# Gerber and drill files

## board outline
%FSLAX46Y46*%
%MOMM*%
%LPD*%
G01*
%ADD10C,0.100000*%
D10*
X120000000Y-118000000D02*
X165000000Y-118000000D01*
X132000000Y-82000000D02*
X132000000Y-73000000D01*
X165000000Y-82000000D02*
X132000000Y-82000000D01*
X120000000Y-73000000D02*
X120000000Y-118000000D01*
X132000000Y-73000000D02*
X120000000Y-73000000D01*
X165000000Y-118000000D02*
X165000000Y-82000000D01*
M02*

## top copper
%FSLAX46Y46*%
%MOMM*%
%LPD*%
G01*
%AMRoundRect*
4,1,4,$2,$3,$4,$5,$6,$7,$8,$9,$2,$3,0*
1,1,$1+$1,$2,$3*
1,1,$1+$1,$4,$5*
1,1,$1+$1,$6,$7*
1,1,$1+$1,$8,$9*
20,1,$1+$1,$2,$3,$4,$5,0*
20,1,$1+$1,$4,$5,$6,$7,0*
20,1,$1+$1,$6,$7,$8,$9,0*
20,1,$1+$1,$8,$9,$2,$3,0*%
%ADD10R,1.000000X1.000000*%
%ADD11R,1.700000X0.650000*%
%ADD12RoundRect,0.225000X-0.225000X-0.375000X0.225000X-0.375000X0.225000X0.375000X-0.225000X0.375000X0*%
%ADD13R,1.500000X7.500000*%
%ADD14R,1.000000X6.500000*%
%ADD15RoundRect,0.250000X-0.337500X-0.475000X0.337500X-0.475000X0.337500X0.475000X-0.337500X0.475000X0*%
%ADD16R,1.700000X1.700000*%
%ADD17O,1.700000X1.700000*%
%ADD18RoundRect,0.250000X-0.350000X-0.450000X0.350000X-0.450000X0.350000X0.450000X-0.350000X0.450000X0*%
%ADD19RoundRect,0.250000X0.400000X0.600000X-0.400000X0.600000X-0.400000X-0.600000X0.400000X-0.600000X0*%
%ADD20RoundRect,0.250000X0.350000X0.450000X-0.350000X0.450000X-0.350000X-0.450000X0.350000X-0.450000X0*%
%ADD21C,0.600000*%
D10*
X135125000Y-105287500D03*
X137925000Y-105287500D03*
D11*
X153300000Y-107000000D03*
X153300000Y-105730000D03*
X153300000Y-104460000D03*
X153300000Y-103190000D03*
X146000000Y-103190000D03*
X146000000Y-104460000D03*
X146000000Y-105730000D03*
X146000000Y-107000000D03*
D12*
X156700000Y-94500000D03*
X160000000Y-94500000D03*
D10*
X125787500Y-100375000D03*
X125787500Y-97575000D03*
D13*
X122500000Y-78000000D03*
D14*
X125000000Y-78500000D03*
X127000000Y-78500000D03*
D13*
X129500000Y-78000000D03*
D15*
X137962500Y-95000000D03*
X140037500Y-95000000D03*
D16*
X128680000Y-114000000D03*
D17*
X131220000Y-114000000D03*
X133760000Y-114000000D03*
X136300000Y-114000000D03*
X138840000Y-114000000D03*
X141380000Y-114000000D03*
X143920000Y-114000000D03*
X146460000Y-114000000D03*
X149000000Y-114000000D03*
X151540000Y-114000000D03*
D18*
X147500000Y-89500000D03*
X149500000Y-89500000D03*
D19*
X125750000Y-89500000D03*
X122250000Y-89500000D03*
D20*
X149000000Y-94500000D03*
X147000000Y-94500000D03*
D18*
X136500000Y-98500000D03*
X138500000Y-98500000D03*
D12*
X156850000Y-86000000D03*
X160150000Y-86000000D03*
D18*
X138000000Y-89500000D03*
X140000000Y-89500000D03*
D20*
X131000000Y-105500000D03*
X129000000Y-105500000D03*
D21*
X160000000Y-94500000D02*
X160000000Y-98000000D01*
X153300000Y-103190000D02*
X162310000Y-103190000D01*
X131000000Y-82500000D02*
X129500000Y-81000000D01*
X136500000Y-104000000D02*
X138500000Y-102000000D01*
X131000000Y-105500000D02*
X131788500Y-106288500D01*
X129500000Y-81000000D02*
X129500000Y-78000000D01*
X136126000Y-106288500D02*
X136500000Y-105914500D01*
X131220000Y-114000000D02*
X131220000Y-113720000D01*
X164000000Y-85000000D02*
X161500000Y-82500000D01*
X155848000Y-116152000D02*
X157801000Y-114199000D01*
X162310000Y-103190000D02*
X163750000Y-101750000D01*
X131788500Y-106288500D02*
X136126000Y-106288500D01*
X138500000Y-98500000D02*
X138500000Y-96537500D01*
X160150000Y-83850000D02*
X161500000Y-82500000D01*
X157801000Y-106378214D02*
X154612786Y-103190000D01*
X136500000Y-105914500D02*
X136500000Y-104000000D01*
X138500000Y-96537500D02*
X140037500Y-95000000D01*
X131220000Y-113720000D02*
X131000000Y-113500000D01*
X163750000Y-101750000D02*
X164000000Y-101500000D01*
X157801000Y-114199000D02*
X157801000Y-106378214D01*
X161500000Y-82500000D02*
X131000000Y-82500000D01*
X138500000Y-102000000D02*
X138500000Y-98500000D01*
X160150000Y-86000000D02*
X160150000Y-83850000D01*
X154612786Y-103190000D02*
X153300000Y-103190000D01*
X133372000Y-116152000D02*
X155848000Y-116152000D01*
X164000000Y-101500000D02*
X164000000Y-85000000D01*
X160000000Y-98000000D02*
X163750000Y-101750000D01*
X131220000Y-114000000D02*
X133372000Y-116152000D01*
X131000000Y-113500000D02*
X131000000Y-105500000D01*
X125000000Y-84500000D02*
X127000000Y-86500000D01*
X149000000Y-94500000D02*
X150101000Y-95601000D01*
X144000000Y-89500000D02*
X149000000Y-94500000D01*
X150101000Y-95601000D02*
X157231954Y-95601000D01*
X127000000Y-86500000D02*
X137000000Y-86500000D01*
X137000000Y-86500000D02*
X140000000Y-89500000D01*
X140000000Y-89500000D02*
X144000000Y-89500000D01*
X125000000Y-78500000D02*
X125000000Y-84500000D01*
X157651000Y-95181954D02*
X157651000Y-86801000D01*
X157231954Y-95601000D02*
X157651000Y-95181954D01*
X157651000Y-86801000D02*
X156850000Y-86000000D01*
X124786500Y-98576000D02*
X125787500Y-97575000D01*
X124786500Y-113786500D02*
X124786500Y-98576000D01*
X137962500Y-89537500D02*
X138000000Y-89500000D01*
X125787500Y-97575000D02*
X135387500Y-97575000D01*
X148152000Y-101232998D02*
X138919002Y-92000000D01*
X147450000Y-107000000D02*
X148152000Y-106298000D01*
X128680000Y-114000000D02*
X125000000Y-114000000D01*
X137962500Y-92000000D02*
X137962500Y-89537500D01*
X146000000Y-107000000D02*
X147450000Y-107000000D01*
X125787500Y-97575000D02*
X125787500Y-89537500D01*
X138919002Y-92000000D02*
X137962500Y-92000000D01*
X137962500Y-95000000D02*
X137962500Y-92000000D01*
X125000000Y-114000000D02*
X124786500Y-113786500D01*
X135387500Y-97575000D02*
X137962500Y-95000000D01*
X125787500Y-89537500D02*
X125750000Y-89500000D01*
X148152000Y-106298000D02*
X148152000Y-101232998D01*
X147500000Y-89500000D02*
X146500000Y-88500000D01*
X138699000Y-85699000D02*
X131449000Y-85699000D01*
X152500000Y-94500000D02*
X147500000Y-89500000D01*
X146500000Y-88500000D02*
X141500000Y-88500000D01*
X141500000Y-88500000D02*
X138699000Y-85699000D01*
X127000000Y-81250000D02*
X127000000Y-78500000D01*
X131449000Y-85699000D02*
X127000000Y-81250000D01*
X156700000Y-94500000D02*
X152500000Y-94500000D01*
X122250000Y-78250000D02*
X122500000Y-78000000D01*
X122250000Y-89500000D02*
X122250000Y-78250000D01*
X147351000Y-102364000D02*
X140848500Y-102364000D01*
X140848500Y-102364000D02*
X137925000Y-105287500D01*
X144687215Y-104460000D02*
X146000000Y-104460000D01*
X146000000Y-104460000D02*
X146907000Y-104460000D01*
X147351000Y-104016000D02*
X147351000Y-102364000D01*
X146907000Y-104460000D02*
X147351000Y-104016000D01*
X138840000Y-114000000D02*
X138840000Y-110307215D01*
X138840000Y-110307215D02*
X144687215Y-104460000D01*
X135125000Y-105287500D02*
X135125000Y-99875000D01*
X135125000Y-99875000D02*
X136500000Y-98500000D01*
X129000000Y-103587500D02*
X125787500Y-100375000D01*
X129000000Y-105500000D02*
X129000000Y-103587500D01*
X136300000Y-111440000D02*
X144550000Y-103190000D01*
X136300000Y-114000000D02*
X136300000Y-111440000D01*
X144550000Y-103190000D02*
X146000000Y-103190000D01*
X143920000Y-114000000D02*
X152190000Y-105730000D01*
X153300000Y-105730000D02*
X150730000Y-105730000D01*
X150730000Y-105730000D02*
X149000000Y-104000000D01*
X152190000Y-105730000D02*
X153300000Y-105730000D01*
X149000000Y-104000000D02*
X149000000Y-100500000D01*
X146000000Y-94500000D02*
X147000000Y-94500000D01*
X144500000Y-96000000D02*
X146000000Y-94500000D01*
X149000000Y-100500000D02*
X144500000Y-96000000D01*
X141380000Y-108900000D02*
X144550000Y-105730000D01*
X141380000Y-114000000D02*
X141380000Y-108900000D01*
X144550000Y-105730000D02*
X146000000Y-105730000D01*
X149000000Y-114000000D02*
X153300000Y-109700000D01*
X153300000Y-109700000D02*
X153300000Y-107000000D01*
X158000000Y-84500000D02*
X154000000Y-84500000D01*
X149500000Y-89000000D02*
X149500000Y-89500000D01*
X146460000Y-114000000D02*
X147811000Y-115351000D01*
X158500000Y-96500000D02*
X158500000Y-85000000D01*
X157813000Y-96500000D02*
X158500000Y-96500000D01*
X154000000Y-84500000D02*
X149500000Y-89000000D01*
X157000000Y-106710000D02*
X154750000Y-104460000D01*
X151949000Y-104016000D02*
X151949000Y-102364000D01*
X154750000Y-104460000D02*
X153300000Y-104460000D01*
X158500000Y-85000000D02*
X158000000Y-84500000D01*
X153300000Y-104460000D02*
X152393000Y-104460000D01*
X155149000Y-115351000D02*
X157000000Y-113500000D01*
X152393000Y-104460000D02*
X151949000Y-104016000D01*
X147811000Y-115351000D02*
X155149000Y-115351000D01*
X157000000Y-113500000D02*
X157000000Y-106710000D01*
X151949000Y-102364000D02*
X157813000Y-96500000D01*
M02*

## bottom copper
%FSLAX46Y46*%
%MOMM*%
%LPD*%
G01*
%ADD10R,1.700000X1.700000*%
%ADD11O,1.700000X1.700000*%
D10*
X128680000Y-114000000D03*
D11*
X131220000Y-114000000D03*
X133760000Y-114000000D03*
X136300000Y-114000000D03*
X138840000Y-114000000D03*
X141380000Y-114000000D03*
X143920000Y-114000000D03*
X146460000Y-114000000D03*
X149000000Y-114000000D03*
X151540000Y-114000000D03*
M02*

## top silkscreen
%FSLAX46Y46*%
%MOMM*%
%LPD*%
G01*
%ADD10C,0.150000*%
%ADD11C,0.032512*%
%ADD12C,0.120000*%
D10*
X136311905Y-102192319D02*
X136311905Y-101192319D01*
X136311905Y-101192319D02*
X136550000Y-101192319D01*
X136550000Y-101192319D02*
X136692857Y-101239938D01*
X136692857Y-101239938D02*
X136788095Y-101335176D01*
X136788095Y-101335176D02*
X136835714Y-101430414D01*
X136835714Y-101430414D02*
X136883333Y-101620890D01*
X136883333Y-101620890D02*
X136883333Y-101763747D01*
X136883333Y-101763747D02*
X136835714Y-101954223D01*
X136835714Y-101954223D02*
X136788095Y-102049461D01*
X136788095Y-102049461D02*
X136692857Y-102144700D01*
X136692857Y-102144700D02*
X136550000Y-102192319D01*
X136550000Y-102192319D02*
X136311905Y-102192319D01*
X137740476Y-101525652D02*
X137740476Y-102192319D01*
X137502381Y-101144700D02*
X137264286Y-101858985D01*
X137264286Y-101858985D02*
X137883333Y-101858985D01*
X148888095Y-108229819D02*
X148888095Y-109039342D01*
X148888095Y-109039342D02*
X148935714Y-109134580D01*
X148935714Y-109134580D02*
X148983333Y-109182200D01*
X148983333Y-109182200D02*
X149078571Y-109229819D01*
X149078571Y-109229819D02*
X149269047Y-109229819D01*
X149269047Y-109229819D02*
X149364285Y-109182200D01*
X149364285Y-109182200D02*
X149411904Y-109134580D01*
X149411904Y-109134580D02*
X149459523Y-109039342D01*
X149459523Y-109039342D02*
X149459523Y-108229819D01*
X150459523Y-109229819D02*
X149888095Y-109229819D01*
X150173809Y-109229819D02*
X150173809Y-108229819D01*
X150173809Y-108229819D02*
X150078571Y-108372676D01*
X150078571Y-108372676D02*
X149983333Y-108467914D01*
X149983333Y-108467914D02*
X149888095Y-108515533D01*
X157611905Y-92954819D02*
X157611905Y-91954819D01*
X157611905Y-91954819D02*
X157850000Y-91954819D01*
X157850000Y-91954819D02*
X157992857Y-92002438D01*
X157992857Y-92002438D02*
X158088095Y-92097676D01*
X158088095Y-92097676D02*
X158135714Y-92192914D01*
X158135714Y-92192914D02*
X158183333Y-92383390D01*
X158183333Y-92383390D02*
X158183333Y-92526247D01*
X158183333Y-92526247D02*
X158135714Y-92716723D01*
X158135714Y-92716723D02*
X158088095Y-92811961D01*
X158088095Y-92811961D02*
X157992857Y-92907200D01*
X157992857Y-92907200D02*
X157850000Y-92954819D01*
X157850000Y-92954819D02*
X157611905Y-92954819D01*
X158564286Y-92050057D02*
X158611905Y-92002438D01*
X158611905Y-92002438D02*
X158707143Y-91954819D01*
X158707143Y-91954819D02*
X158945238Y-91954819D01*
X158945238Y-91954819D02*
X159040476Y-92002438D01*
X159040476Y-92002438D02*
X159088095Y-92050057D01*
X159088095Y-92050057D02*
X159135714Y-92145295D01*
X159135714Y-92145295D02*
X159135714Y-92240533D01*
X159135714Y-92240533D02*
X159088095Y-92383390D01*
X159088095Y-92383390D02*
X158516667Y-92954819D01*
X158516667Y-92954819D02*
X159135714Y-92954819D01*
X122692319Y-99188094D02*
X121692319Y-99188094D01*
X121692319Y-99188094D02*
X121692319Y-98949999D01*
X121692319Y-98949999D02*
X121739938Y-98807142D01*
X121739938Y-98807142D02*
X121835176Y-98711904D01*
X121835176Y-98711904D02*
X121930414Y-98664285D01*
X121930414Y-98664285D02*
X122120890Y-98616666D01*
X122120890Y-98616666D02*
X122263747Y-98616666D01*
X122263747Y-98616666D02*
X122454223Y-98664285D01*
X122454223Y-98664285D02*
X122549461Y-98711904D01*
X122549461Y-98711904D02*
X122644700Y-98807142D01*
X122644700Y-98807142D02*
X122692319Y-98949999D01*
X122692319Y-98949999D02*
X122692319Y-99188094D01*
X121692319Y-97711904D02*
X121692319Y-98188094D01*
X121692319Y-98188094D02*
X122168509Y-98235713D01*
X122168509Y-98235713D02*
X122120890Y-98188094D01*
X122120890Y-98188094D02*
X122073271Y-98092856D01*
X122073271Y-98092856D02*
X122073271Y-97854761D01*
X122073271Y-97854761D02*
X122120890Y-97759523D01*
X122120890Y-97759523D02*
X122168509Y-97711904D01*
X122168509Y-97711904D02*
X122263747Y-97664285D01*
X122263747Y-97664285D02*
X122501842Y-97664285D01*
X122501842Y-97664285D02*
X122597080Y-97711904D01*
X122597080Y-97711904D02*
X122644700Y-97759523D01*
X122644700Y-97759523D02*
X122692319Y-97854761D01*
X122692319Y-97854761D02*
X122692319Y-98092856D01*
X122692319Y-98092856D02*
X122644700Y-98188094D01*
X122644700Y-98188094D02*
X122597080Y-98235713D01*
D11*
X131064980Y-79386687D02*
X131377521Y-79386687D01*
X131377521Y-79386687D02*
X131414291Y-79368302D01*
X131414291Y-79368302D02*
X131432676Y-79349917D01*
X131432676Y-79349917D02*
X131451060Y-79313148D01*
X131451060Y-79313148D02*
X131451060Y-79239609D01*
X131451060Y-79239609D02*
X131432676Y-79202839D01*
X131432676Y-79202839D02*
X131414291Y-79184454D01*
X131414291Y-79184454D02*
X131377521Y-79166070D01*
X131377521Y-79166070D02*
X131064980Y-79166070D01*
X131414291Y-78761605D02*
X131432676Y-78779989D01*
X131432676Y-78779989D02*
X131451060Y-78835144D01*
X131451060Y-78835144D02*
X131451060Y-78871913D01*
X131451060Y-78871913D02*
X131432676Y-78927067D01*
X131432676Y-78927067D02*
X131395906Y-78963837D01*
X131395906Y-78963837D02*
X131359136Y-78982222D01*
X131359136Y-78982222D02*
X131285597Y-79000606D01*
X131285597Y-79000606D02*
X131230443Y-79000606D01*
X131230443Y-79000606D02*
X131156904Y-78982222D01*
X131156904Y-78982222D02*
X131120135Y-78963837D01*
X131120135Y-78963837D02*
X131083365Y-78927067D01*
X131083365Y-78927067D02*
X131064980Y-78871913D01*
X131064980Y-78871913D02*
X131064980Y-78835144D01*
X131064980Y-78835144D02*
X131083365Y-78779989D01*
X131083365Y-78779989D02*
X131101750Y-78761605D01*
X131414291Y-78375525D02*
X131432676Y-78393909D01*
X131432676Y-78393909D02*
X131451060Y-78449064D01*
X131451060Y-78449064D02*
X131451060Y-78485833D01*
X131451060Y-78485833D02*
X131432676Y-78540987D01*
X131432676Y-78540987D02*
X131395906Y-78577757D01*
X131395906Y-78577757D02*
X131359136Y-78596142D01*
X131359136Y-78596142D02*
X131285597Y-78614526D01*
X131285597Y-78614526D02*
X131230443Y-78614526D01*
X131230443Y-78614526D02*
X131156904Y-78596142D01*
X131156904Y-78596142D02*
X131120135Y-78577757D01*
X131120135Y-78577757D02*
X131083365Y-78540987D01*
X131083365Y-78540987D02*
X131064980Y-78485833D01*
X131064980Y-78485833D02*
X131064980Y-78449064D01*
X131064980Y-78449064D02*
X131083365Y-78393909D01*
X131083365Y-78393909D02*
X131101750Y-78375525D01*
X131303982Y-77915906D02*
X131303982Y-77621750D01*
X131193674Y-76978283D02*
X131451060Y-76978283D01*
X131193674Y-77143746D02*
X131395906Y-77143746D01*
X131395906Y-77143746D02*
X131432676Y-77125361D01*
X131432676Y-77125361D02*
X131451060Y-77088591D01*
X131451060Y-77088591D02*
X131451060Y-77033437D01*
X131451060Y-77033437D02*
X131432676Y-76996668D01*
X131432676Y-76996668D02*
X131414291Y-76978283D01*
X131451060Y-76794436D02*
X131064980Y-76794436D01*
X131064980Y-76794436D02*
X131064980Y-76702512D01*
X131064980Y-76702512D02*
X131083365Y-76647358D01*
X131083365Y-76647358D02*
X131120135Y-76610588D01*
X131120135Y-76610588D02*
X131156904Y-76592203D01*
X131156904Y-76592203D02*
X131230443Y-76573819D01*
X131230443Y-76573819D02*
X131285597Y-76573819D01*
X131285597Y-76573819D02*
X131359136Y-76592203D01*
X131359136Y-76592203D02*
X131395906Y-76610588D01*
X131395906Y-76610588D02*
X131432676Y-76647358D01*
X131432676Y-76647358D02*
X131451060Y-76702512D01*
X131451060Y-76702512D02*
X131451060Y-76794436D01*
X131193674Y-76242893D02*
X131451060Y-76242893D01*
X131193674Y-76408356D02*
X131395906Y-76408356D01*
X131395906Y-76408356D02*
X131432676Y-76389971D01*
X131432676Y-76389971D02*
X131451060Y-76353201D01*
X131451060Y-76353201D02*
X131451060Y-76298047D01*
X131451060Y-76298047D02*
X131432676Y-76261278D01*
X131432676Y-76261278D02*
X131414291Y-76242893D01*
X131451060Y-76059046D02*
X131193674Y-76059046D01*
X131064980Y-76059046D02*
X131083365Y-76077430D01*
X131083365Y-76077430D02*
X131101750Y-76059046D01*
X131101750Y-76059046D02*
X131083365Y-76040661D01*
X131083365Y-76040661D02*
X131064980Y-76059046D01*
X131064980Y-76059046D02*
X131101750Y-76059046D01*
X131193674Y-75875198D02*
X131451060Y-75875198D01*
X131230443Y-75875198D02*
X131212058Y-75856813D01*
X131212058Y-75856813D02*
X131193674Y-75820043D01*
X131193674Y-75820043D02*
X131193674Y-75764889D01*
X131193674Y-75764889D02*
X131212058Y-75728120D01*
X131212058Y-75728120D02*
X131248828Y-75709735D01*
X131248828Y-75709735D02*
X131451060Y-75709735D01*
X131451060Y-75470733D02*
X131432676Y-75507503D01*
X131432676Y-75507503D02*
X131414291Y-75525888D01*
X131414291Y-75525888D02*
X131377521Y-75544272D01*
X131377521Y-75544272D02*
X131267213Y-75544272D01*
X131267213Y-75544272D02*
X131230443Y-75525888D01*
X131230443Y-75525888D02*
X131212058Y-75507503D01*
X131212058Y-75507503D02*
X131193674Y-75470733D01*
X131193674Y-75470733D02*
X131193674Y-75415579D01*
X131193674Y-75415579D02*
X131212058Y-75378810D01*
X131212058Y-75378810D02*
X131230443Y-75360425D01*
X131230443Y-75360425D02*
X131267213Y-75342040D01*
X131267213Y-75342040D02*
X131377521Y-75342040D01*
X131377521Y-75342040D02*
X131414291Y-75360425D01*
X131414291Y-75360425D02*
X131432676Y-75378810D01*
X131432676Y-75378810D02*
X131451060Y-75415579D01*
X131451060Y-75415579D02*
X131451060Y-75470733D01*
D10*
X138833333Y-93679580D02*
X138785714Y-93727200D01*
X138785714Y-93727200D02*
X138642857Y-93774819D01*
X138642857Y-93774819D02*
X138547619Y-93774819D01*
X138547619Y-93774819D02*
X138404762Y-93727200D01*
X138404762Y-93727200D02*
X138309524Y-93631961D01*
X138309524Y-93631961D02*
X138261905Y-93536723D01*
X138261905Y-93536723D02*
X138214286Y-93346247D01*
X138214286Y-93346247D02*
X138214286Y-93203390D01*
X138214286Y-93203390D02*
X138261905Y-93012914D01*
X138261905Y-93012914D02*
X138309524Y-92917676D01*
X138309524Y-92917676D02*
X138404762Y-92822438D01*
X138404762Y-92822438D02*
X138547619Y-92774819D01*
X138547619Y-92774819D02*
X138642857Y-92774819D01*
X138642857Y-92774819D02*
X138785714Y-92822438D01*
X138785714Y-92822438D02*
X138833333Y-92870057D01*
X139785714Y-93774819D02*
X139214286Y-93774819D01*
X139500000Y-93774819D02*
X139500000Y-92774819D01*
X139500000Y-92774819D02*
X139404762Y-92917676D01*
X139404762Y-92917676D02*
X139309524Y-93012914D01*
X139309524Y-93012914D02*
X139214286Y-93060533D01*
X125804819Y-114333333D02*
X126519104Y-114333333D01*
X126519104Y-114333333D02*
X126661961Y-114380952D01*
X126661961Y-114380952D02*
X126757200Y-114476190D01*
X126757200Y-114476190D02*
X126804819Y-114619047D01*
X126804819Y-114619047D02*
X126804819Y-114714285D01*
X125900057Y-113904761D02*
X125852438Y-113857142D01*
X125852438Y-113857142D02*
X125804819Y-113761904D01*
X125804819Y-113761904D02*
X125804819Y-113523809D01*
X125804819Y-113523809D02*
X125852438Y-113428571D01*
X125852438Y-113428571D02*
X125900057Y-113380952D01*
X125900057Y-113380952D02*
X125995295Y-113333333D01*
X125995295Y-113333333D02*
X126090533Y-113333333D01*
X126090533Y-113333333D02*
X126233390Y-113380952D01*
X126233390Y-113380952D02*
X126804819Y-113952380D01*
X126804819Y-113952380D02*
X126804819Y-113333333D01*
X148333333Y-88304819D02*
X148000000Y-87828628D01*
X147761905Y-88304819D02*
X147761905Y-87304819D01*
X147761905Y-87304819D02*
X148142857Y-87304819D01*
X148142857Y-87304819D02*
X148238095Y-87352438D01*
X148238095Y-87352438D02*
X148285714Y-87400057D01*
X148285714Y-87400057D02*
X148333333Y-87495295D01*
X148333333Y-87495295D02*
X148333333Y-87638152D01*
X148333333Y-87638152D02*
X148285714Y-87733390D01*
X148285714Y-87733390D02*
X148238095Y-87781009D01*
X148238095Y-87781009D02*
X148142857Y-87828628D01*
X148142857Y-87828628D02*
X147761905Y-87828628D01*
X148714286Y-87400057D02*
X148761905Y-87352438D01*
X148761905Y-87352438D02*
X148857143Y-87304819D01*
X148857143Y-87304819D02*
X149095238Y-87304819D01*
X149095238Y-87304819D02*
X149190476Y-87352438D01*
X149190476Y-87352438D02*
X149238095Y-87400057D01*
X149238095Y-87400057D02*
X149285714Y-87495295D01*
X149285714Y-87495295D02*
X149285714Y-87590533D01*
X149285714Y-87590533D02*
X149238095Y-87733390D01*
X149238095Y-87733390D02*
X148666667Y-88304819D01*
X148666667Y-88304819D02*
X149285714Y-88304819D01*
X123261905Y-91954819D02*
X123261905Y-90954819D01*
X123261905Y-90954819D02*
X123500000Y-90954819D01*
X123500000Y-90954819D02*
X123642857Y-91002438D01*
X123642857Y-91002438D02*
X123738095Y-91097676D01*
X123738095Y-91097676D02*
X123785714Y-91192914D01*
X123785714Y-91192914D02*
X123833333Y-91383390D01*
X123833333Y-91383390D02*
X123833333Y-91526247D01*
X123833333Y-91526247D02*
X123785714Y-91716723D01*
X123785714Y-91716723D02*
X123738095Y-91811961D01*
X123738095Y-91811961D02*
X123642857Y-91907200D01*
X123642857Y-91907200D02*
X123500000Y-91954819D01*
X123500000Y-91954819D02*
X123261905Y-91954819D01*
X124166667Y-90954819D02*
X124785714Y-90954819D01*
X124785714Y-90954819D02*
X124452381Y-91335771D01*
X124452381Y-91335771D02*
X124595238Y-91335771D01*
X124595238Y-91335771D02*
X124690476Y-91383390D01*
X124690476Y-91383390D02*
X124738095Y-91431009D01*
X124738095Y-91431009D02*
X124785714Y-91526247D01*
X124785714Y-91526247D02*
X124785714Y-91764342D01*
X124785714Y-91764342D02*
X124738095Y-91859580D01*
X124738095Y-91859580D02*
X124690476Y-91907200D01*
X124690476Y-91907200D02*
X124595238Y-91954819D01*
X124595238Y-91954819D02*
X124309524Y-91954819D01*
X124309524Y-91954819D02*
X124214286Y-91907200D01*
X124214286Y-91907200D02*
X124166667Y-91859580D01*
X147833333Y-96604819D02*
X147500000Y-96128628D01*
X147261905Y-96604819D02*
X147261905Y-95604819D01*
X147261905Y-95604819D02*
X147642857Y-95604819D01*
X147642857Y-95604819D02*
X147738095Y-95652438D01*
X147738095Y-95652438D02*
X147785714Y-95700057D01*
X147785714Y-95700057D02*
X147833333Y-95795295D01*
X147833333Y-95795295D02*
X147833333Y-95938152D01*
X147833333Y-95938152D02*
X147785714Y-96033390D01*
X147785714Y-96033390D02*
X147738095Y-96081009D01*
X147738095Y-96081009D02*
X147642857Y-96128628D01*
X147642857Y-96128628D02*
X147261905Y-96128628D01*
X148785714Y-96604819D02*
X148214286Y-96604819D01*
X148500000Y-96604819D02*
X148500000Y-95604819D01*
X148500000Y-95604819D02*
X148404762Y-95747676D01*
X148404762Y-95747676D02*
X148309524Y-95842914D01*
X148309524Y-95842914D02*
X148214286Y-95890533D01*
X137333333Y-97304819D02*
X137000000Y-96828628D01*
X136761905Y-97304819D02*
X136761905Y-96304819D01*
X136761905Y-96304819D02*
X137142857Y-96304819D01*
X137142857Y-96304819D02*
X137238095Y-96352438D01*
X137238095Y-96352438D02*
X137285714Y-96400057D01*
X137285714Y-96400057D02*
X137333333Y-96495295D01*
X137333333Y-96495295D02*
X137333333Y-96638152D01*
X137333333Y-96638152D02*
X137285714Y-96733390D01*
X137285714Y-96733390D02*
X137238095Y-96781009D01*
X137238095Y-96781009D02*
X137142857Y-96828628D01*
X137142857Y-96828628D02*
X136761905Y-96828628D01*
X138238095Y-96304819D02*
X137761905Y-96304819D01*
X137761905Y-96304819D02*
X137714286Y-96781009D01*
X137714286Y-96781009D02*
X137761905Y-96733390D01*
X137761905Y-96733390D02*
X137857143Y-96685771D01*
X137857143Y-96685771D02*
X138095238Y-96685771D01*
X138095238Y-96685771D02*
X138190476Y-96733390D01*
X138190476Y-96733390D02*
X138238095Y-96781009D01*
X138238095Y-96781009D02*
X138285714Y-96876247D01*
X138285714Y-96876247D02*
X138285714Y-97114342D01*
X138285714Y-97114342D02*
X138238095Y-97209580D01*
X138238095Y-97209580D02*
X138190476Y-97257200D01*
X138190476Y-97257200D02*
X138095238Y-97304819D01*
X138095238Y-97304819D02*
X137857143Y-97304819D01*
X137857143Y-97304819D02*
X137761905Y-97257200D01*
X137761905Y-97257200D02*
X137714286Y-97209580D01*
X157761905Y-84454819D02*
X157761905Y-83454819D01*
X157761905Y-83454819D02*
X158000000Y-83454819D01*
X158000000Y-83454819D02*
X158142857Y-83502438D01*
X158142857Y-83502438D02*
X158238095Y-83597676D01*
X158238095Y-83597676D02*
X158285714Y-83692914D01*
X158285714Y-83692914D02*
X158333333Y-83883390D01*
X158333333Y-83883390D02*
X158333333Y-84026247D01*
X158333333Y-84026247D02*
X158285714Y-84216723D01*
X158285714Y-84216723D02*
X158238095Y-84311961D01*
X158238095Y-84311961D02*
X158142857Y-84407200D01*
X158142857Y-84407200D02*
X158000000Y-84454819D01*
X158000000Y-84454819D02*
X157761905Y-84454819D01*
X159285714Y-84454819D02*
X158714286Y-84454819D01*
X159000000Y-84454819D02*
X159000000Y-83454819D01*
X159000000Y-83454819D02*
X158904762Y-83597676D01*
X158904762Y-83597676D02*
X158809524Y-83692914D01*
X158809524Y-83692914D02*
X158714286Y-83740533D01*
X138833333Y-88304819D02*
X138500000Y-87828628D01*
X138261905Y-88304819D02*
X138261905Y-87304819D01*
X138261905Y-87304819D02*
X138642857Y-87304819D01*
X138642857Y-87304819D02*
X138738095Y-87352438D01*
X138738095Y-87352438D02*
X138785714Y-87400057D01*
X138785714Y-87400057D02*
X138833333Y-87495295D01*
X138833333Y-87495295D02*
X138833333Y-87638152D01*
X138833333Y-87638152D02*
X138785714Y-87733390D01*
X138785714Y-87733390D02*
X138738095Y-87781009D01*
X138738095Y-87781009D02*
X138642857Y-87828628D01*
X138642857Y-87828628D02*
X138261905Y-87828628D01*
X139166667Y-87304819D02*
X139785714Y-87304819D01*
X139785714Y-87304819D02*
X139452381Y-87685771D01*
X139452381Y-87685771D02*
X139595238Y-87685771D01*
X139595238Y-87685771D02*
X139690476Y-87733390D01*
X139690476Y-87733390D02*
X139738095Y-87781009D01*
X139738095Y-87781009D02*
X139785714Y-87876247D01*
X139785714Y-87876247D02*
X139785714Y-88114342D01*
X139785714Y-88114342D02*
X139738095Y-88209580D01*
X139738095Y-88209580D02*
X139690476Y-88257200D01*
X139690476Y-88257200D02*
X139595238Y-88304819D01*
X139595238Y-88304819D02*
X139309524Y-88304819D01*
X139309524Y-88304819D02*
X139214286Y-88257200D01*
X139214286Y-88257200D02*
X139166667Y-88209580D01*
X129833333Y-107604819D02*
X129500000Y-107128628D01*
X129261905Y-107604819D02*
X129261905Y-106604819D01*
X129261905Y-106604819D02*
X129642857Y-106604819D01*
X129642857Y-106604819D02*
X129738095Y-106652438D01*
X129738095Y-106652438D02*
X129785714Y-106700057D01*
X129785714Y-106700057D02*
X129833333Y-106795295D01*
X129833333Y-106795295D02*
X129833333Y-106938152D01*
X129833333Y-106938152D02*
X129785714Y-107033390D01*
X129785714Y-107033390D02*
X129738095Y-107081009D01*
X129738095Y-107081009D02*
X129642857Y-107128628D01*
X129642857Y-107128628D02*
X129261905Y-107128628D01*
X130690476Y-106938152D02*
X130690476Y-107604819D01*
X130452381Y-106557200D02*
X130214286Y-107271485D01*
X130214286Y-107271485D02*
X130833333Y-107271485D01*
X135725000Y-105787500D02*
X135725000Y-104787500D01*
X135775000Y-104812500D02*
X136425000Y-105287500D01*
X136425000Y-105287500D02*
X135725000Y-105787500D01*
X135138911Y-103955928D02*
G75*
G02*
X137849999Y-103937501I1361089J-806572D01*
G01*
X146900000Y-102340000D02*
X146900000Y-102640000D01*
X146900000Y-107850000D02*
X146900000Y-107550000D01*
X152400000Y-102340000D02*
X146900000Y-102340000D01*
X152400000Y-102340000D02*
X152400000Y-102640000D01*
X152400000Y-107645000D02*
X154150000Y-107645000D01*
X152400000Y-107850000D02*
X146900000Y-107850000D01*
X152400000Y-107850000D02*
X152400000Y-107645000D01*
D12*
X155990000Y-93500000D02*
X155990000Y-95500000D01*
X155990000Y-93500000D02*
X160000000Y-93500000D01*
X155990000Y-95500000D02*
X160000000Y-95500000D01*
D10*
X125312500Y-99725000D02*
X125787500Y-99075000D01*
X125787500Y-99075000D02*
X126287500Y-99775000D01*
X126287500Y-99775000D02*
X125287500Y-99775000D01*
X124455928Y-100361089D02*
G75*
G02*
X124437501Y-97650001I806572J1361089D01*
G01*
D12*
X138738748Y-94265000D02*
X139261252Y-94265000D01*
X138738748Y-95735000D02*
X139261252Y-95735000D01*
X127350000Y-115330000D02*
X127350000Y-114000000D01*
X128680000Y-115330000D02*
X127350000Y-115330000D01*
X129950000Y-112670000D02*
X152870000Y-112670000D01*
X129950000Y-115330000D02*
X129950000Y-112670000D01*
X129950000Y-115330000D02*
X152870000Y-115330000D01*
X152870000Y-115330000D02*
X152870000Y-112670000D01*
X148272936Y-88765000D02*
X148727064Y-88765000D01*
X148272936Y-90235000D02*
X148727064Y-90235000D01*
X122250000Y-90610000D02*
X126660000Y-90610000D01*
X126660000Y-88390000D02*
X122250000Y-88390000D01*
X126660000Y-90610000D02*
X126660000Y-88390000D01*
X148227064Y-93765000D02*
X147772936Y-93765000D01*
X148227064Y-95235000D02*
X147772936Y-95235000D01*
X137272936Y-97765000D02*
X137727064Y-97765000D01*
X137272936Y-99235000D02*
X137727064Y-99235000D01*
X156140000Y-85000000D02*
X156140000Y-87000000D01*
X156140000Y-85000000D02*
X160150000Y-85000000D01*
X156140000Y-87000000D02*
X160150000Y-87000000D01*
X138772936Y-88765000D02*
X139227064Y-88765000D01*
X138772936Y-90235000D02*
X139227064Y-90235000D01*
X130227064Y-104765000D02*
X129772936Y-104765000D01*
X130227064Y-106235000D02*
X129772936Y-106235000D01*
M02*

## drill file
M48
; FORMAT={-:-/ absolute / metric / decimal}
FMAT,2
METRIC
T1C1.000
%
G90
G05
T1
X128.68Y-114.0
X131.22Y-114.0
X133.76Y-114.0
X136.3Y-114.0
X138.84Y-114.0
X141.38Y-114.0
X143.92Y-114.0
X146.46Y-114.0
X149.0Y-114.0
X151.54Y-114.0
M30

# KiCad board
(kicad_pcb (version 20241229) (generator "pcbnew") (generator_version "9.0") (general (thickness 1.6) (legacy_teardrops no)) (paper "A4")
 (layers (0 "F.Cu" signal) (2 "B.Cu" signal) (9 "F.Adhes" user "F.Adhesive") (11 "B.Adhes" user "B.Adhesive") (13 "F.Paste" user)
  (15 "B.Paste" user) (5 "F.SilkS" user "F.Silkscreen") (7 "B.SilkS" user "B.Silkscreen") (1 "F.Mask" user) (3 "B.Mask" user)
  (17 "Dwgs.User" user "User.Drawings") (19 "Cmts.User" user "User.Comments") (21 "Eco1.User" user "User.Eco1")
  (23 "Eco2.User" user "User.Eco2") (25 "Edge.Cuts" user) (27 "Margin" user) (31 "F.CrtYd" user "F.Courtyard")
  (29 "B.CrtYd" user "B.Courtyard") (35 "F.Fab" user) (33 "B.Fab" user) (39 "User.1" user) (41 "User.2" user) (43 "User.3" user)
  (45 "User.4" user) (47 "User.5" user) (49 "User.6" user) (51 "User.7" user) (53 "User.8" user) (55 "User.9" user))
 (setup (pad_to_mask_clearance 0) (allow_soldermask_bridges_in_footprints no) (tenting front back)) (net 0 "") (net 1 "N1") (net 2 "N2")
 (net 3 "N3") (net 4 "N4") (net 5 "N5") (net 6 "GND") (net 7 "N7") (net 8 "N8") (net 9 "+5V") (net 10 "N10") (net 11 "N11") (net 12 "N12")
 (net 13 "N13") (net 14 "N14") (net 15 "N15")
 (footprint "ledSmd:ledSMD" (layer "F.Cu") (at 136.925 105.2875)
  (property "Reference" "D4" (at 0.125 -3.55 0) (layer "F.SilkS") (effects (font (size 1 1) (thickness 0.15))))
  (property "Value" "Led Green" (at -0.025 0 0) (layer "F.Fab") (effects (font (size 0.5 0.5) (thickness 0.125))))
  (fp_line (start -1.2 0.5) (end -1.2 -0.5) (stroke (width 0.15) (type solid)) (layer "F.SilkS"))
  (fp_line (start -1.15 -0.475) (end -0.5 0) (stroke (width 0.15) (type solid)) (layer "F.SilkS"))
  (fp_line (start -0.5 0) (end -1.2 0.5) (stroke (width 0.15) (type solid)) (layer "F.SilkS"))
  (fp_arc (start -1.786089 -1.331572) (mid -0.435753 -2.107089) (end 0.924999 -1.349999) (stroke (width 0.15) (type solid))
   (layer "F.SilkS"))
  (pad "1" smd rect (at -1.8 0) (size 1 1) (layers "F.Cu" "F.Mask" "F.Paste") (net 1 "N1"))
  (pad "2" smd rect (at 1 0) (size 1 1) (layers "F.Cu" "F.Mask" "F.Paste") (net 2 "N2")))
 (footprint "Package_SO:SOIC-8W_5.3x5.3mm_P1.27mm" (layer "F.Cu") (at 149.65 105.095 180)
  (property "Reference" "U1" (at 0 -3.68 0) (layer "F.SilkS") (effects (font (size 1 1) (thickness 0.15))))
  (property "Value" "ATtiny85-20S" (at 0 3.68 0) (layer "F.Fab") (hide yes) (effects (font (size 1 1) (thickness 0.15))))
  (fp_line (start 2.75 2.755) (end 2.75 2.455) (stroke (width 0.15) (type solid)) (layer "F.SilkS"))
  (fp_line (start 2.75 -2.755) (end 2.75 -2.455) (stroke (width 0.15) (type solid)) (layer "F.SilkS"))
  (fp_line (start -2.75 2.755) (end 2.75 2.755) (stroke (width 0.15) (type solid)) (layer "F.SilkS"))
  (fp_line (start -2.75 2.755) (end -2.75 2.455) (stroke (width 0.15) (type solid)) (layer "F.SilkS"))
  (fp_line (start -2.75 -2.55) (end -4.5 -2.55) (stroke (width 0.15) (type solid)) (layer "F.SilkS"))
  (fp_line (start -2.75 -2.755) (end 2.75 -2.755) (stroke (width 0.15) (type solid)) (layer "F.SilkS"))
  (fp_line (start -2.75 -2.755) (end -2.75 -2.55) (stroke (width 0.15) (type solid)) (layer "F.SilkS"))
  (pad "1" smd rect (at -3.65 -1.905 180) (size 1.7 0.65) (layers "F.Cu" "F.Mask" "F.Paste") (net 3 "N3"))
  (pad "2" smd rect (at -3.65 -0.635 180) (size 1.7 0.65) (layers "F.Cu" "F.Mask" "F.Paste") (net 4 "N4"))
  (pad "3" smd rect (at -3.65 0.635 180) (size 1.7 0.65) (layers "F.Cu" "F.Mask" "F.Paste") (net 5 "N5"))
  (pad "4" smd rect (at -3.65 1.905 180) (size 1.7 0.65) (layers "F.Cu" "F.Mask" "F.Paste") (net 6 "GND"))
  (pad "5" smd rect (at 3.65 1.905 180) (size 1.7 0.65) (layers "F.Cu" "F.Mask" "F.Paste") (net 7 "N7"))
  (pad "6" smd rect (at 3.65 0.635 180) (size 1.7 0.65) (layers "F.Cu" "F.Mask" "F.Paste") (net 2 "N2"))
  (pad "7" smd rect (at 3.65 -0.635 180) (size 1.7 0.65) (layers "F.Cu" "F.Mask" "F.Paste") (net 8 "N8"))
  (pad "8" smd rect (at 3.65 -1.905 180) (size 1.7 0.65) (layers "F.Cu" "F.Mask" "F.Paste") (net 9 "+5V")))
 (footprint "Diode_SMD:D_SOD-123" (layer "F.Cu") (at 158.35 94.5)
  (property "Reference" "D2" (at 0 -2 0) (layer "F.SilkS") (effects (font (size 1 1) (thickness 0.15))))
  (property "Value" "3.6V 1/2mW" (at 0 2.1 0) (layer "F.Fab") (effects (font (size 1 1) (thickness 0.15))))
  (fp_line (start -2.36 -1) (end -2.36 1) (stroke (width 0.12) (type solid)) (layer "F.SilkS"))
  (fp_line (start -2.36 -1) (end 1.65 -1) (stroke (width 0.12) (type solid)) (layer "F.SilkS"))
  (fp_line (start -2.36 1) (end 1.65 1) (stroke (width 0.12) (type solid)) (layer "F.SilkS"))
  (pad "1" smd roundrect (at -1.65 0) (size 0.9 1.2) (layers "F.Cu" "F.Mask" "F.Paste") (roundrect_rratio 0.25) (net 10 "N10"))
  (pad "2" smd roundrect (at 1.65 0) (size 0.9 1.2) (layers "F.Cu" "F.Mask" "F.Paste") (roundrect_rratio 0.25) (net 6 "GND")))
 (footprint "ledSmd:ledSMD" (layer "F.Cu") (at 125.7875 98.575 90)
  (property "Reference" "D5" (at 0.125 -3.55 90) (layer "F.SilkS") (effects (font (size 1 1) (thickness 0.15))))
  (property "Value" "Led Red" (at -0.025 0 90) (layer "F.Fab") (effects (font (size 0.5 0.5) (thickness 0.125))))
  (fp_line (start -1.15 -0.475) (end -0.5 0) (stroke (width 0.15) (type solid)) (layer "F.SilkS"))
  (fp_line (start -0.5 0) (end -1.2 0.5) (stroke (width 0.15) (type solid)) (layer "F.SilkS"))
  (fp_line (start -1.2 0.5) (end -1.2 -0.5) (stroke (width 0.15) (type solid)) (layer "F.SilkS"))
  (fp_arc (start -1.786089 -1.331572) (mid -0.435753 -2.107089) (end 0.924999 -1.349999) (stroke (width 0.15) (type solid))
   (layer "F.SilkS"))
  (pad "1" smd rect (at -1.8 0 90) (size 1 1) (layers "F.Cu" "F.Mask" "F.Paste") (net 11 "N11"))
  (pad "2" smd rect (at 1 0 90) (size 1 1) (layers "F.Cu" "F.Mask" "F.Paste") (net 9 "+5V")))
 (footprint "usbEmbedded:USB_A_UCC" (layer "F.Cu") (at 126 78.2 -90)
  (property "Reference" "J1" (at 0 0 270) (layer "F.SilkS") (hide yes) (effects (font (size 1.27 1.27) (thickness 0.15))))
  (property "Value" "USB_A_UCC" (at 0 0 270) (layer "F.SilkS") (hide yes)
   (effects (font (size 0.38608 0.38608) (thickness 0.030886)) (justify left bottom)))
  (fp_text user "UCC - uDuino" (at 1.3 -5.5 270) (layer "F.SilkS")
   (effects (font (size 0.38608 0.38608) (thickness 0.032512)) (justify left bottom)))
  (pad "1" smd rect (at -0.2 3.5 270) (size 7.5 1.5) (layers "F.Cu" "F.Mask" "F.Paste") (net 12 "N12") (solder_mask_margin 0.1016))
  (pad "2" smd rect (at 0.3 1 270) (size 6.5 1) (layers "F.Cu" "F.Mask" "F.Paste") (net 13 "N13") (solder_mask_margin 0.1016))
  (pad "3" smd rect (at 0.3 -1 270) (size 6.5 1) (layers "F.Cu" "F.Mask" "F.Paste") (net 10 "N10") (solder_mask_margin 0.1016))
  (pad "4" smd rect (at -0.2 -3.5 270) (size 7.5 1.5) (layers "F.Cu" "F.Mask" "F.Paste") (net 6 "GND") (solder_mask_margin 0.1016)))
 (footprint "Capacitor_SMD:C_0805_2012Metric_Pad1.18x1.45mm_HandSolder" (layer "F.Cu") (at 139 95)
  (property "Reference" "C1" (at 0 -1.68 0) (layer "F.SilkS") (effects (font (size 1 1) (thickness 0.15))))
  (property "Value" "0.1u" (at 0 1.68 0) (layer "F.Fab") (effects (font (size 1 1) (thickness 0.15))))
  (fp_line (start -0.261252 -0.735) (end 0.261252 -0.735) (stroke (width 0.12) (type solid)) (layer "F.SilkS"))
  (fp_line (start -0.261252 0.735) (end 0.261252 0.735) (stroke (width 0.12) (type solid)) (layer "F.SilkS"))
  (pad "1" smd roundrect (at -1.0375 0) (size 1.175 1.45) (layers "F.Cu" "F.Mask" "F.Paste") (roundrect_rratio 0.212766) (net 9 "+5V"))
  (pad "2" smd roundrect (at 1.0375 0) (size 1.175 1.45) (layers "F.Cu" "F.Mask" "F.Paste") (roundrect_rratio 0.212766) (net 6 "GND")))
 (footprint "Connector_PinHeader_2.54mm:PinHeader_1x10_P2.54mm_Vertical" (layer "F.Cu") (at 128.68 114 90)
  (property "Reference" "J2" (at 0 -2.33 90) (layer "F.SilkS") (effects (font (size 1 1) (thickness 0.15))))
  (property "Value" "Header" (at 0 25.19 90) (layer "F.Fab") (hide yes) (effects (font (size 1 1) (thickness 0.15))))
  (fp_line (start -1.33 -1.33) (end 0 -1.33) (stroke (width 0.12) (type solid)) (layer "F.SilkS"))
  (fp_line (start -1.33 0) (end -1.33 -1.33) (stroke (width 0.12) (type solid)) (layer "F.SilkS"))
  (fp_line (start 1.33 1.27) (end 1.33 24.19) (stroke (width 0.12) (type solid)) (layer "F.SilkS"))
  (fp_line (start -1.33 1.27) (end 1.33 1.27) (stroke (width 0.12) (type solid)) (layer "F.SilkS"))
  (fp_line (start -1.33 1.27) (end -1.33 24.19) (stroke (width 0.12) (type solid)) (layer "F.SilkS"))
  (fp_line (start -1.33 24.19) (end 1.33 24.19) (stroke (width 0.12) (type solid)) (layer "F.SilkS"))
  (pad "1" thru_hole rect (at 0 0 90) (size 1.7 1.7) (drill 1) (layers "*.Cu" "*.Mask") (remove_unused_layers no) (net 9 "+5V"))
  (pad "2" thru_hole oval (at 0 2.54 90) (size 1.7 1.7) (drill 1) (layers "*.Cu" "*.Mask") (remove_unused_layers no) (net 6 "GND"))
  (pad "3" thru_hole oval (at 0 5.08 90) (size 1.7 1.7) (drill 1) (layers "*.Cu" "*.Mask") (remove_unused_layers no) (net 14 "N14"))
  (pad "4" thru_hole oval (at 0 7.62 90) (size 1.7 1.7) (drill 1) (layers "*.Cu" "*.Mask") (remove_unused_layers no) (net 7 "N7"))
  (pad "5" thru_hole oval (at 0 10.16 90) (size 1.7 1.7) (drill 1) (layers "*.Cu" "*.Mask") (remove_unused_layers no) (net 2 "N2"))
  (pad "6" thru_hole oval (at 0 12.7 90) (size 1.7 1.7) (drill 1) (layers "*.Cu" "*.Mask") (remove_unused_layers no) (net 8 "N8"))
  (pad "7" thru_hole oval (at 0 15.24 90) (size 1.7 1.7) (drill 1) (layers "*.Cu" "*.Mask") (remove_unused_layers no) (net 4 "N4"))
  (pad "8" thru_hole oval (at 0 17.78 90) (size 1.7 1.7) (drill 1) (layers "*.Cu" "*.Mask") (remove_unused_layers no) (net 5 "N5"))
  (pad "9" thru_hole oval (at 0 20.32 90) (size 1.7 1.7) (drill 1) (layers "*.Cu" "*.Mask") (remove_unused_layers no) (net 3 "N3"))
  (pad "10" thru_hole oval (at 0 22.86 90) (size 1.7 1.7) (drill 1) (layers "*.Cu" "*.Mask") (remove_unused_layers no) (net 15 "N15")))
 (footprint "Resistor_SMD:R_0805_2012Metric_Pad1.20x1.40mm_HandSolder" (layer "F.Cu") (at 148.5 89.5)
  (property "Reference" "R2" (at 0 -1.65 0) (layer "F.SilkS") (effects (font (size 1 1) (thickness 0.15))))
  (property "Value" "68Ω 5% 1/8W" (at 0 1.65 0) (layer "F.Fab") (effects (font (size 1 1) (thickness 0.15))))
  (fp_line (start -0.227064 -0.735) (end 0.227064 -0.735) (stroke (width 0.12) (type solid)) (layer "F.SilkS"))
  (fp_line (start -0.227064 0.735) (end 0.227064 0.735) (stroke (width 0.12) (type solid)) (layer "F.SilkS"))
  (pad "1" smd roundrect (at -1 0) (size 1.2 1.4) (layers "F.Cu" "F.Mask" "F.Paste") (roundrect_rratio 0.208333) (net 10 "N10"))
  (pad "2" smd roundrect (at 1 0) (size 1.2 1.4) (layers "F.Cu" "F.Mask" "F.Paste") (roundrect_rratio 0.208333) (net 5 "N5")))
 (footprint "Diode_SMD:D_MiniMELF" (layer "F.Cu") (at 124 89.5 180)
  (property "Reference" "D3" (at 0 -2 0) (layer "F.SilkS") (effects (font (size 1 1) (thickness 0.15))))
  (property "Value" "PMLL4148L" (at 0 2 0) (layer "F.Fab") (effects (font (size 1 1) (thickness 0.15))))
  (fp_line (start 1.75 -1.11) (end -2.66 -1.11) (stroke (width 0.12) (type solid)) (layer "F.SilkS"))
  (fp_line (start -2.66 1.11) (end 1.75 1.11) (stroke (width 0.12) (type solid)) (layer "F.SilkS"))
  (fp_line (start -2.66 -1.11) (end -2.66 1.11) (stroke (width 0.12) (type solid)) (layer "F.SilkS"))
  (pad "1" smd roundrect (at -1.75 0 180) (size 1.3 1.7) (layers "F.Cu" "F.Mask" "F.Paste") (roundrect_rratio 0.1923076923) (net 9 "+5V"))
  (pad "2" smd roundrect (at 1.75 0 180) (size 1.3 1.7) (layers "F.Cu" "F.Mask" "F.Paste") (roundrect_rratio 0.1923076923) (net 12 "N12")))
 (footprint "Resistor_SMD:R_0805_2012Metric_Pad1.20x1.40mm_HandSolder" (layer "F.Cu") (at 148 94.5 180)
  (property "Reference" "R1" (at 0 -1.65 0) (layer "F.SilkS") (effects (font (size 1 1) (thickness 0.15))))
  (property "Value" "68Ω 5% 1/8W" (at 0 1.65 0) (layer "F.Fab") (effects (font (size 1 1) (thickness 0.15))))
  (fp_line (start -0.227064 0.735) (end 0.227064 0.735) (stroke (width 0.12) (type solid)) (layer "F.SilkS"))
  (fp_line (start -0.227064 -0.735) (end 0.227064 -0.735) (stroke (width 0.12) (type solid)) (layer "F.SilkS"))
  (pad "1" smd roundrect (at -1 0 180) (size 1.2 1.4) (layers "F.Cu" "F.Mask" "F.Paste") (roundrect_rratio 0.208333) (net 13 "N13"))
  (pad "2" smd roundrect (at 1 0 180) (size 1.2 1.4) (layers "F.Cu" "F.Mask" "F.Paste") (roundrect_rratio 0.208333) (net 4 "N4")))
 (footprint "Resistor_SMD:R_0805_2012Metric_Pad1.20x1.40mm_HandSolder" (layer "F.Cu") (at 137.5 98.5)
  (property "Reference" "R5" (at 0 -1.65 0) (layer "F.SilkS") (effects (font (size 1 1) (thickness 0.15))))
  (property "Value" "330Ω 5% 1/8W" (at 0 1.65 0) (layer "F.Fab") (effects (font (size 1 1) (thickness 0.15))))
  (fp_line (start -0.227064 -0.735) (end 0.227064 -0.735) (stroke (width 0.12) (type solid)) (layer "F.SilkS"))
  (fp_line (start -0.227064 0.735) (end 0.227064 0.735) (stroke (width 0.12) (type solid)) (layer "F.SilkS"))
  (pad "1" smd roundrect (at -1 0) (size 1.2 1.4) (layers "F.Cu" "F.Mask" "F.Paste") (roundrect_rratio 0.208333) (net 1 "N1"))
  (pad "2" smd roundrect (at 1 0) (size 1.2 1.4) (layers "F.Cu" "F.Mask" "F.Paste") (roundrect_rratio 0.208333) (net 6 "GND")))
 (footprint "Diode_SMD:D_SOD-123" (layer "F.Cu") (at 158.5 86)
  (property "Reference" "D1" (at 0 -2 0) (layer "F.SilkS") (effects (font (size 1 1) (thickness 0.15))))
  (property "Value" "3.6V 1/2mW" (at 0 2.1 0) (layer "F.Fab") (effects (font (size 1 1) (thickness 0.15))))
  (fp_line (start -2.36 -1) (end -2.36 1) (stroke (width 0.12) (type solid)) (layer "F.SilkS"))
  (fp_line (start -2.36 -1) (end 1.65 -1) (stroke (width 0.12) (type solid)) (layer "F.SilkS"))
  (fp_line (start -2.36 1) (end 1.65 1) (stroke (width 0.12) (type solid)) (layer "F.SilkS"))
  (pad "1" smd roundrect (at -1.65 0) (size 0.9 1.2) (layers "F.Cu" "F.Mask" "F.Paste") (roundrect_rratio 0.25) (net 13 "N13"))
  (pad "2" smd roundrect (at 1.65 0) (size 0.9 1.2) (layers "F.Cu" "F.Mask" "F.Paste") (roundrect_rratio 0.25) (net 6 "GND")))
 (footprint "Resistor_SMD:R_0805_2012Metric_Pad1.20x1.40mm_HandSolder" (layer "F.Cu") (at 139 89.5)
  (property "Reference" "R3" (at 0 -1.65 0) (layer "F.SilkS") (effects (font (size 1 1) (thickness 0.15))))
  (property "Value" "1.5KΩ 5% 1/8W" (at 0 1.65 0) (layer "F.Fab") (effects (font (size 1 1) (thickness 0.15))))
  (fp_line (start -0.227064 -0.735) (end 0.227064 -0.735) (stroke (width 0.12) (type solid)) (layer "F.SilkS"))
  (fp_line (start -0.227064 0.735) (end 0.227064 0.735) (stroke (width 0.12) (type solid)) (layer "F.SilkS"))
  (pad "1" smd roundrect (at -1 0) (size 1.2 1.4) (layers "F.Cu" "F.Mask" "F.Paste") (roundrect_rratio 0.208333) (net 9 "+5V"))
  (pad "2" smd roundrect (at 1 0) (size 1.2 1.4) (layers "F.Cu" "F.Mask" "F.Paste") (roundrect_rratio 0.208333) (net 13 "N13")))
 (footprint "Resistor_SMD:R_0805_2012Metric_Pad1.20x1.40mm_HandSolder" (layer "F.Cu") (at 130 105.5 180)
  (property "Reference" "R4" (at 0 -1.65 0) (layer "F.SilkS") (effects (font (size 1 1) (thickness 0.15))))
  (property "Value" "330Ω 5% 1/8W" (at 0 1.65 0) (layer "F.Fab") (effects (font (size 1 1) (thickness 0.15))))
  (fp_line (start -0.227064 0.735) (end 0.227064 0.735) (stroke (width 0.12) (type solid)) (layer "F.SilkS"))
  (fp_line (start -0.227064 -0.735) (end 0.227064 -0.735) (stroke (width 0.12) (type solid)) (layer "F.SilkS"))
  (pad "1" smd roundrect (at -1 0 180) (size 1.2 1.4) (layers "F.Cu" "F.Mask" "F.Paste") (roundrect_rratio 0.208333) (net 6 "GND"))
  (pad "2" smd roundrect (at 1 0 180) (size 1.2 1.4) (layers "F.Cu" "F.Mask" "F.Paste") (roundrect_rratio 0.208333) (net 11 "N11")))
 (gr_line (start 120 118) (end 165 118) (stroke (width 0.1) (type default)) (layer "Edge.Cuts"))
 (gr_line (start 132 82) (end 132 73) (stroke (width 0.1) (type default)) (layer "Edge.Cuts"))
 (gr_line (start 165 82) (end 132 82) (stroke (width 0.1) (type default)) (layer "Edge.Cuts"))
 (gr_line (start 120 73) (end 120 118) (stroke (width 0.1) (type default)) (layer "Edge.Cuts"))
 (gr_line (start 132 73) (end 120 73) (stroke (width 0.1) (type default)) (layer "Edge.Cuts"))
 (gr_line (start 165 118) (end 165 82) (stroke (width 0.1) (type default)) (layer "Edge.Cuts"))
 (segment (start 160 94.5) (end 160 98) (width 0.6) (layer "F.Cu") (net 6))
 (segment (start 153.3 103.19) (end 162.31 103.19) (width 0.6) (layer "F.Cu") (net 6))
 (segment (start 131 82.5) (end 129.5 81) (width 0.6) (layer "F.Cu") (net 6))
 (segment (start 136.5 104) (end 138.5 102) (width 0.6) (layer "F.Cu") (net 6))
 (segment (start 131 105.5) (end 131.7885 106.2885) (width 0.6) (layer "F.Cu") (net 6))
 (segment (start 129.5 81) (end 129.5 78) (width 0.6) (layer "F.Cu") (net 6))
 (segment (start 136.126 106.2885) (end 136.5 105.9145) (width 0.6) (layer "F.Cu") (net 6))
 (segment (start 131.22 114) (end 131.22 113.72) (width 0.6) (layer "F.Cu") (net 6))
 (segment (start 164 85) (end 161.5 82.5) (width 0.6) (layer "F.Cu") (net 6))
 (segment (start 155.848 116.152) (end 157.801 114.199) (width 0.6) (layer "F.Cu") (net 6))
 (segment (start 162.31 103.19) (end 163.75 101.75) (width 0.6) (layer "F.Cu") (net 6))
 (segment (start 131.7885 106.2885) (end 136.126 106.2885) (width 0.6) (layer "F.Cu") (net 6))
 (segment (start 138.5 98.5) (end 138.5 96.5375) (width 0.6) (layer "F.Cu") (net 6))
 (segment (start 160.15 83.85) (end 161.5 82.5) (width 0.6) (layer "F.Cu") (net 6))
 (segment (start 157.801 106.378214) (end 154.612786 103.19) (width 0.6) (layer "F.Cu") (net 6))
 (segment (start 136.5 105.9145) (end 136.5 104) (width 0.6) (layer "F.Cu") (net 6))
 (segment (start 138.5 96.5375) (end 140.0375 95) (width 0.6) (layer "F.Cu") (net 6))
 (segment (start 131.22 113.72) (end 131 113.5) (width 0.6) (layer "F.Cu") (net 6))
 (segment (start 163.75 101.75) (end 164 101.5) (width 0.6) (layer "F.Cu") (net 6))
 (segment (start 157.801 114.199) (end 157.801 106.378214) (width 0.6) (layer "F.Cu") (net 6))
 (segment (start 161.5 82.5) (end 131 82.5) (width 0.6) (layer "F.Cu") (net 6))
 (segment (start 138.5 102) (end 138.5 98.5) (width 0.6) (layer "F.Cu") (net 6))
 (segment (start 160.15 86) (end 160.15 83.85) (width 0.6) (layer "F.Cu") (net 6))
 (segment (start 154.612786 103.19) (end 153.3 103.19) (width 0.6) (layer "F.Cu") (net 6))
 (segment (start 133.372 116.152) (end 155.848 116.152) (width 0.6) (layer "F.Cu") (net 6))
 (segment (start 164 101.5) (end 164 85) (width 0.6) (layer "F.Cu") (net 6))
 (segment (start 160 98) (end 163.75 101.75) (width 0.6) (layer "F.Cu") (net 6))
 (segment (start 131.22 114) (end 133.372 116.152) (width 0.6) (layer "F.Cu") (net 6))
 (segment (start 131 113.5) (end 131 105.5) (width 0.6) (layer "F.Cu") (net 6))
 (segment (start 125 84.5) (end 127 86.5) (width 0.6) (layer "F.Cu") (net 13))
 (segment (start 149 94.5) (end 150.101 95.601) (width 0.6) (layer "F.Cu") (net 13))
 (segment (start 144 89.5) (end 149 94.5) (width 0.6) (layer "F.Cu") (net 13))
 (segment (start 150.101 95.601) (end 157.231954 95.601) (width 0.6) (layer "F.Cu") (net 13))
 (segment (start 127 86.5) (end 137 86.5) (width 0.6) (layer "F.Cu") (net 13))
 (segment (start 137 86.5) (end 140 89.5) (width 0.6) (layer "F.Cu") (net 13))
 (segment (start 140 89.5) (end 144 89.5) (width 0.6) (layer "F.Cu") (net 13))
 (segment (start 125 78.5) (end 125 84.5) (width 0.6) (layer "F.Cu") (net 13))
 (segment (start 157.651 95.181954) (end 157.651 86.801) (width 0.6) (layer "F.Cu") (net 13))
 (segment (start 157.231954 95.601) (end 157.651 95.181954) (width 0.6) (layer "F.Cu") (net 13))
 (segment (start 157.651 86.801) (end 156.85 86) (width 0.6) (layer "F.Cu") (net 13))
 (segment (start 124.7865 98.576) (end 125.7875 97.575) (width 0.6) (layer "F.Cu") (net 9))
 (segment (start 124.7865 113.7865) (end 124.7865 98.576) (width 0.6) (layer "F.Cu") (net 9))
 (segment (start 137.9625 89.5375) (end 138 89.5) (width 0.6) (layer "F.Cu") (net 9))
 (segment (start 125.7875 97.575) (end 135.3875 97.575) (width 0.6) (layer "F.Cu") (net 9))
 (segment (start 148.152 101.232998) (end 138.919002 92) (width 0.6) (layer "F.Cu") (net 9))
 (segment (start 147.45 107) (end 148.152 106.298) (width 0.6) (layer "F.Cu") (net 9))
 (segment (start 128.68 114) (end 125 114) (width 0.6) (layer "F.Cu") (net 9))
 (segment (start 137.9625 92) (end 137.9625 89.5375) (width 0.6) (layer "F.Cu") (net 9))
 (segment (start 146 107) (end 147.45 107) (width 0.6) (layer "F.Cu") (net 9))
 (segment (start 125.7875 97.575) (end 125.7875 89.5375) (width 0.6) (layer "F.Cu") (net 9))
 (segment (start 138.919002 92) (end 137.9625 92) (width 0.6) (layer "F.Cu") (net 9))
 (segment (start 137.9625 95) (end 137.9625 92) (width 0.6) (layer "F.Cu") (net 9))
 (segment (start 125 114) (end 124.7865 113.7865) (width 0.6) (layer "F.Cu") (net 9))
 (segment (start 135.3875 97.575) (end 137.9625 95) (width 0.6) (layer "F.Cu") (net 9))
 (segment (start 125.7875 89.5375) (end 125.75 89.5) (width 0.6) (layer "F.Cu") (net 9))
 (segment (start 148.152 106.298) (end 148.152 101.232998) (width 0.6) (layer "F.Cu") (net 9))
 (segment (start 147.5 89.5) (end 146.5 88.5) (width 0.6) (layer "F.Cu") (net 10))
 (segment (start 138.699 85.699) (end 131.449 85.699) (width 0.6) (layer "F.Cu") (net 10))
 (segment (start 152.5 94.5) (end 147.5 89.5) (width 0.6) (layer "F.Cu") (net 10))
 (segment (start 146.5 88.5) (end 141.5 88.5) (width 0.6) (layer "F.Cu") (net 10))
 (segment (start 141.5 88.5) (end 138.699 85.699) (width 0.6) (layer "F.Cu") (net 10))
 (segment (start 127 81.25) (end 127 78.5) (width 0.6) (layer "F.Cu") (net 10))
 (segment (start 131.449 85.699) (end 127 81.25) (width 0.6) (layer "F.Cu") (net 10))
 (segment (start 156.7 94.5) (end 152.5 94.5) (width 0.6) (layer "F.Cu") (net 10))
 (segment (start 122.25 78.25) (end 122.5 78) (width 0.6) (layer "F.Cu") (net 12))
 (segment (start 122.25 89.5) (end 122.25 78.25) (width 0.6) (layer "F.Cu") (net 12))
 (segment (start 147.351 102.364) (end 140.8485 102.364) (width 0.6) (layer "F.Cu") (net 2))
 (segment (start 140.8485 102.364) (end 137.925 105.2875) (width 0.6) (layer "F.Cu") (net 2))
 (segment (start 144.687215 104.46) (end 146 104.46) (width 0.6) (layer "F.Cu") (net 2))
 (segment (start 146 104.46) (end 146.907 104.46) (width 0.6) (layer "F.Cu") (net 2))
 (segment (start 147.351 104.016) (end 147.351 102.364) (width 0.6) (layer "F.Cu") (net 2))
 (segment (start 146.907 104.46) (end 147.351 104.016) (width 0.6) (layer "F.Cu") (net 2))
 (segment (start 138.84 114) (end 138.84 110.307215) (width 0.6) (layer "F.Cu") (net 2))
 (segment (start 138.84 110.307215) (end 144.687215 104.46) (width 0.6) (layer "F.Cu") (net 2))
 (segment (start 135.125 105.2875) (end 135.125 99.875) (width 0.6) (layer "F.Cu") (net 1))
 (segment (start 135.125 99.875) (end 136.5 98.5) (width 0.6) (layer "F.Cu") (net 1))
 (segment (start 129 103.5875) (end 125.7875 100.375) (width 0.6) (layer "F.Cu") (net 11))
 (segment (start 129 105.5) (end 129 103.5875) (width 0.6) (layer "F.Cu") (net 11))
 (segment (start 136.3 111.44) (end 144.55 103.19) (width 0.6) (layer "F.Cu") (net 7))
 (segment (start 136.3 114) (end 136.3 111.44) (width 0.6) (layer "F.Cu") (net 7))
 (segment (start 144.55 103.19) (end 146 103.19) (width 0.6) (layer "F.Cu") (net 7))
 (segment (start 143.92 114) (end 152.19 105.73) (width 0.6) (layer "F.Cu") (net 4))
 (segment (start 153.3 105.73) (end 150.73 105.73) (width 0.6) (layer "F.Cu") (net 4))
 (segment (start 150.73 105.73) (end 149 104) (width 0.6) (layer "F.Cu") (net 4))
 (segment (start 152.19 105.73) (end 153.3 105.73) (width 0.6) (layer "F.Cu") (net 4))
 (segment (start 149 104) (end 149 100.5) (width 0.6) (layer "F.Cu") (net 4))
 (segment (start 146 94.5) (end 147 94.5) (width 0.6) (layer "F.Cu") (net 4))
 (segment (start 144.5 96) (end 146 94.5) (width 0.6) (layer "F.Cu") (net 4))
 (segment (start 149 100.5) (end 144.5 96) (width 0.6) (layer "F.Cu") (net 4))
 (segment (start 141.38 108.9) (end 144.55 105.73) (width 0.6) (layer "F.Cu") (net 8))
 (segment (start 141.38 114) (end 141.38 108.9) (width 0.6) (layer "F.Cu") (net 8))
 (segment (start 144.55 105.73) (end 146 105.73) (width 0.6) (layer "F.Cu") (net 8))
 (segment (start 149 114) (end 153.3 109.7) (width 0.6) (layer "F.Cu") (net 3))
 (segment (start 153.3 109.7) (end 153.3 107) (width 0.6) (layer "F.Cu") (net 3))
 (segment (start 158 84.5) (end 154 84.5) (width 0.6) (layer "F.Cu") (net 5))
 (segment (start 149.5 89) (end 149.5 89.5) (width 0.6) (layer "F.Cu") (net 5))
 (segment (start 146.46 114) (end 147.811 115.351) (width 0.6) (layer "F.Cu") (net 5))
 (segment (start 158.5 96.5) (end 158.5 85) (width 0.6) (layer "F.Cu") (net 5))
 (segment (start 157.813 96.5) (end 158.5 96.5) (width 0.6) (layer "F.Cu") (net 5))
 (segment (start 154 84.5) (end 149.5 89) (width 0.6) (layer "F.Cu") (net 5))
 (segment (start 157 106.71) (end 154.75 104.46) (width 0.6) (layer "F.Cu") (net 5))
 (segment (start 151.949 104.016) (end 151.949 102.364) (width 0.6) (layer "F.Cu") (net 5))
 (segment (start 154.75 104.46) (end 153.3 104.46) (width 0.6) (layer "F.Cu") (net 5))
 (segment (start 158.5 85) (end 158 84.5) (width 0.6) (layer "F.Cu") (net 5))
 (segment (start 153.3 104.46) (end 152.393 104.46) (width 0.6) (layer "F.Cu") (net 5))
 (segment (start 155.149 115.351) (end 157 113.5) (width 0.6) (layer "F.Cu") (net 5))
 (segment (start 152.393 104.46) (end 151.949 104.016) (width 0.6) (layer "F.Cu") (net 5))
 (segment (start 147.811 115.351) (end 155.149 115.351) (width 0.6) (layer "F.Cu") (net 5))
 (segment (start 157 113.5) (end 157 106.71) (width 0.6) (layer "F.Cu") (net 5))
 (segment (start 151.949 102.364) (end 157.813 96.5) (width 0.6) (layer "F.Cu") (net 5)))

